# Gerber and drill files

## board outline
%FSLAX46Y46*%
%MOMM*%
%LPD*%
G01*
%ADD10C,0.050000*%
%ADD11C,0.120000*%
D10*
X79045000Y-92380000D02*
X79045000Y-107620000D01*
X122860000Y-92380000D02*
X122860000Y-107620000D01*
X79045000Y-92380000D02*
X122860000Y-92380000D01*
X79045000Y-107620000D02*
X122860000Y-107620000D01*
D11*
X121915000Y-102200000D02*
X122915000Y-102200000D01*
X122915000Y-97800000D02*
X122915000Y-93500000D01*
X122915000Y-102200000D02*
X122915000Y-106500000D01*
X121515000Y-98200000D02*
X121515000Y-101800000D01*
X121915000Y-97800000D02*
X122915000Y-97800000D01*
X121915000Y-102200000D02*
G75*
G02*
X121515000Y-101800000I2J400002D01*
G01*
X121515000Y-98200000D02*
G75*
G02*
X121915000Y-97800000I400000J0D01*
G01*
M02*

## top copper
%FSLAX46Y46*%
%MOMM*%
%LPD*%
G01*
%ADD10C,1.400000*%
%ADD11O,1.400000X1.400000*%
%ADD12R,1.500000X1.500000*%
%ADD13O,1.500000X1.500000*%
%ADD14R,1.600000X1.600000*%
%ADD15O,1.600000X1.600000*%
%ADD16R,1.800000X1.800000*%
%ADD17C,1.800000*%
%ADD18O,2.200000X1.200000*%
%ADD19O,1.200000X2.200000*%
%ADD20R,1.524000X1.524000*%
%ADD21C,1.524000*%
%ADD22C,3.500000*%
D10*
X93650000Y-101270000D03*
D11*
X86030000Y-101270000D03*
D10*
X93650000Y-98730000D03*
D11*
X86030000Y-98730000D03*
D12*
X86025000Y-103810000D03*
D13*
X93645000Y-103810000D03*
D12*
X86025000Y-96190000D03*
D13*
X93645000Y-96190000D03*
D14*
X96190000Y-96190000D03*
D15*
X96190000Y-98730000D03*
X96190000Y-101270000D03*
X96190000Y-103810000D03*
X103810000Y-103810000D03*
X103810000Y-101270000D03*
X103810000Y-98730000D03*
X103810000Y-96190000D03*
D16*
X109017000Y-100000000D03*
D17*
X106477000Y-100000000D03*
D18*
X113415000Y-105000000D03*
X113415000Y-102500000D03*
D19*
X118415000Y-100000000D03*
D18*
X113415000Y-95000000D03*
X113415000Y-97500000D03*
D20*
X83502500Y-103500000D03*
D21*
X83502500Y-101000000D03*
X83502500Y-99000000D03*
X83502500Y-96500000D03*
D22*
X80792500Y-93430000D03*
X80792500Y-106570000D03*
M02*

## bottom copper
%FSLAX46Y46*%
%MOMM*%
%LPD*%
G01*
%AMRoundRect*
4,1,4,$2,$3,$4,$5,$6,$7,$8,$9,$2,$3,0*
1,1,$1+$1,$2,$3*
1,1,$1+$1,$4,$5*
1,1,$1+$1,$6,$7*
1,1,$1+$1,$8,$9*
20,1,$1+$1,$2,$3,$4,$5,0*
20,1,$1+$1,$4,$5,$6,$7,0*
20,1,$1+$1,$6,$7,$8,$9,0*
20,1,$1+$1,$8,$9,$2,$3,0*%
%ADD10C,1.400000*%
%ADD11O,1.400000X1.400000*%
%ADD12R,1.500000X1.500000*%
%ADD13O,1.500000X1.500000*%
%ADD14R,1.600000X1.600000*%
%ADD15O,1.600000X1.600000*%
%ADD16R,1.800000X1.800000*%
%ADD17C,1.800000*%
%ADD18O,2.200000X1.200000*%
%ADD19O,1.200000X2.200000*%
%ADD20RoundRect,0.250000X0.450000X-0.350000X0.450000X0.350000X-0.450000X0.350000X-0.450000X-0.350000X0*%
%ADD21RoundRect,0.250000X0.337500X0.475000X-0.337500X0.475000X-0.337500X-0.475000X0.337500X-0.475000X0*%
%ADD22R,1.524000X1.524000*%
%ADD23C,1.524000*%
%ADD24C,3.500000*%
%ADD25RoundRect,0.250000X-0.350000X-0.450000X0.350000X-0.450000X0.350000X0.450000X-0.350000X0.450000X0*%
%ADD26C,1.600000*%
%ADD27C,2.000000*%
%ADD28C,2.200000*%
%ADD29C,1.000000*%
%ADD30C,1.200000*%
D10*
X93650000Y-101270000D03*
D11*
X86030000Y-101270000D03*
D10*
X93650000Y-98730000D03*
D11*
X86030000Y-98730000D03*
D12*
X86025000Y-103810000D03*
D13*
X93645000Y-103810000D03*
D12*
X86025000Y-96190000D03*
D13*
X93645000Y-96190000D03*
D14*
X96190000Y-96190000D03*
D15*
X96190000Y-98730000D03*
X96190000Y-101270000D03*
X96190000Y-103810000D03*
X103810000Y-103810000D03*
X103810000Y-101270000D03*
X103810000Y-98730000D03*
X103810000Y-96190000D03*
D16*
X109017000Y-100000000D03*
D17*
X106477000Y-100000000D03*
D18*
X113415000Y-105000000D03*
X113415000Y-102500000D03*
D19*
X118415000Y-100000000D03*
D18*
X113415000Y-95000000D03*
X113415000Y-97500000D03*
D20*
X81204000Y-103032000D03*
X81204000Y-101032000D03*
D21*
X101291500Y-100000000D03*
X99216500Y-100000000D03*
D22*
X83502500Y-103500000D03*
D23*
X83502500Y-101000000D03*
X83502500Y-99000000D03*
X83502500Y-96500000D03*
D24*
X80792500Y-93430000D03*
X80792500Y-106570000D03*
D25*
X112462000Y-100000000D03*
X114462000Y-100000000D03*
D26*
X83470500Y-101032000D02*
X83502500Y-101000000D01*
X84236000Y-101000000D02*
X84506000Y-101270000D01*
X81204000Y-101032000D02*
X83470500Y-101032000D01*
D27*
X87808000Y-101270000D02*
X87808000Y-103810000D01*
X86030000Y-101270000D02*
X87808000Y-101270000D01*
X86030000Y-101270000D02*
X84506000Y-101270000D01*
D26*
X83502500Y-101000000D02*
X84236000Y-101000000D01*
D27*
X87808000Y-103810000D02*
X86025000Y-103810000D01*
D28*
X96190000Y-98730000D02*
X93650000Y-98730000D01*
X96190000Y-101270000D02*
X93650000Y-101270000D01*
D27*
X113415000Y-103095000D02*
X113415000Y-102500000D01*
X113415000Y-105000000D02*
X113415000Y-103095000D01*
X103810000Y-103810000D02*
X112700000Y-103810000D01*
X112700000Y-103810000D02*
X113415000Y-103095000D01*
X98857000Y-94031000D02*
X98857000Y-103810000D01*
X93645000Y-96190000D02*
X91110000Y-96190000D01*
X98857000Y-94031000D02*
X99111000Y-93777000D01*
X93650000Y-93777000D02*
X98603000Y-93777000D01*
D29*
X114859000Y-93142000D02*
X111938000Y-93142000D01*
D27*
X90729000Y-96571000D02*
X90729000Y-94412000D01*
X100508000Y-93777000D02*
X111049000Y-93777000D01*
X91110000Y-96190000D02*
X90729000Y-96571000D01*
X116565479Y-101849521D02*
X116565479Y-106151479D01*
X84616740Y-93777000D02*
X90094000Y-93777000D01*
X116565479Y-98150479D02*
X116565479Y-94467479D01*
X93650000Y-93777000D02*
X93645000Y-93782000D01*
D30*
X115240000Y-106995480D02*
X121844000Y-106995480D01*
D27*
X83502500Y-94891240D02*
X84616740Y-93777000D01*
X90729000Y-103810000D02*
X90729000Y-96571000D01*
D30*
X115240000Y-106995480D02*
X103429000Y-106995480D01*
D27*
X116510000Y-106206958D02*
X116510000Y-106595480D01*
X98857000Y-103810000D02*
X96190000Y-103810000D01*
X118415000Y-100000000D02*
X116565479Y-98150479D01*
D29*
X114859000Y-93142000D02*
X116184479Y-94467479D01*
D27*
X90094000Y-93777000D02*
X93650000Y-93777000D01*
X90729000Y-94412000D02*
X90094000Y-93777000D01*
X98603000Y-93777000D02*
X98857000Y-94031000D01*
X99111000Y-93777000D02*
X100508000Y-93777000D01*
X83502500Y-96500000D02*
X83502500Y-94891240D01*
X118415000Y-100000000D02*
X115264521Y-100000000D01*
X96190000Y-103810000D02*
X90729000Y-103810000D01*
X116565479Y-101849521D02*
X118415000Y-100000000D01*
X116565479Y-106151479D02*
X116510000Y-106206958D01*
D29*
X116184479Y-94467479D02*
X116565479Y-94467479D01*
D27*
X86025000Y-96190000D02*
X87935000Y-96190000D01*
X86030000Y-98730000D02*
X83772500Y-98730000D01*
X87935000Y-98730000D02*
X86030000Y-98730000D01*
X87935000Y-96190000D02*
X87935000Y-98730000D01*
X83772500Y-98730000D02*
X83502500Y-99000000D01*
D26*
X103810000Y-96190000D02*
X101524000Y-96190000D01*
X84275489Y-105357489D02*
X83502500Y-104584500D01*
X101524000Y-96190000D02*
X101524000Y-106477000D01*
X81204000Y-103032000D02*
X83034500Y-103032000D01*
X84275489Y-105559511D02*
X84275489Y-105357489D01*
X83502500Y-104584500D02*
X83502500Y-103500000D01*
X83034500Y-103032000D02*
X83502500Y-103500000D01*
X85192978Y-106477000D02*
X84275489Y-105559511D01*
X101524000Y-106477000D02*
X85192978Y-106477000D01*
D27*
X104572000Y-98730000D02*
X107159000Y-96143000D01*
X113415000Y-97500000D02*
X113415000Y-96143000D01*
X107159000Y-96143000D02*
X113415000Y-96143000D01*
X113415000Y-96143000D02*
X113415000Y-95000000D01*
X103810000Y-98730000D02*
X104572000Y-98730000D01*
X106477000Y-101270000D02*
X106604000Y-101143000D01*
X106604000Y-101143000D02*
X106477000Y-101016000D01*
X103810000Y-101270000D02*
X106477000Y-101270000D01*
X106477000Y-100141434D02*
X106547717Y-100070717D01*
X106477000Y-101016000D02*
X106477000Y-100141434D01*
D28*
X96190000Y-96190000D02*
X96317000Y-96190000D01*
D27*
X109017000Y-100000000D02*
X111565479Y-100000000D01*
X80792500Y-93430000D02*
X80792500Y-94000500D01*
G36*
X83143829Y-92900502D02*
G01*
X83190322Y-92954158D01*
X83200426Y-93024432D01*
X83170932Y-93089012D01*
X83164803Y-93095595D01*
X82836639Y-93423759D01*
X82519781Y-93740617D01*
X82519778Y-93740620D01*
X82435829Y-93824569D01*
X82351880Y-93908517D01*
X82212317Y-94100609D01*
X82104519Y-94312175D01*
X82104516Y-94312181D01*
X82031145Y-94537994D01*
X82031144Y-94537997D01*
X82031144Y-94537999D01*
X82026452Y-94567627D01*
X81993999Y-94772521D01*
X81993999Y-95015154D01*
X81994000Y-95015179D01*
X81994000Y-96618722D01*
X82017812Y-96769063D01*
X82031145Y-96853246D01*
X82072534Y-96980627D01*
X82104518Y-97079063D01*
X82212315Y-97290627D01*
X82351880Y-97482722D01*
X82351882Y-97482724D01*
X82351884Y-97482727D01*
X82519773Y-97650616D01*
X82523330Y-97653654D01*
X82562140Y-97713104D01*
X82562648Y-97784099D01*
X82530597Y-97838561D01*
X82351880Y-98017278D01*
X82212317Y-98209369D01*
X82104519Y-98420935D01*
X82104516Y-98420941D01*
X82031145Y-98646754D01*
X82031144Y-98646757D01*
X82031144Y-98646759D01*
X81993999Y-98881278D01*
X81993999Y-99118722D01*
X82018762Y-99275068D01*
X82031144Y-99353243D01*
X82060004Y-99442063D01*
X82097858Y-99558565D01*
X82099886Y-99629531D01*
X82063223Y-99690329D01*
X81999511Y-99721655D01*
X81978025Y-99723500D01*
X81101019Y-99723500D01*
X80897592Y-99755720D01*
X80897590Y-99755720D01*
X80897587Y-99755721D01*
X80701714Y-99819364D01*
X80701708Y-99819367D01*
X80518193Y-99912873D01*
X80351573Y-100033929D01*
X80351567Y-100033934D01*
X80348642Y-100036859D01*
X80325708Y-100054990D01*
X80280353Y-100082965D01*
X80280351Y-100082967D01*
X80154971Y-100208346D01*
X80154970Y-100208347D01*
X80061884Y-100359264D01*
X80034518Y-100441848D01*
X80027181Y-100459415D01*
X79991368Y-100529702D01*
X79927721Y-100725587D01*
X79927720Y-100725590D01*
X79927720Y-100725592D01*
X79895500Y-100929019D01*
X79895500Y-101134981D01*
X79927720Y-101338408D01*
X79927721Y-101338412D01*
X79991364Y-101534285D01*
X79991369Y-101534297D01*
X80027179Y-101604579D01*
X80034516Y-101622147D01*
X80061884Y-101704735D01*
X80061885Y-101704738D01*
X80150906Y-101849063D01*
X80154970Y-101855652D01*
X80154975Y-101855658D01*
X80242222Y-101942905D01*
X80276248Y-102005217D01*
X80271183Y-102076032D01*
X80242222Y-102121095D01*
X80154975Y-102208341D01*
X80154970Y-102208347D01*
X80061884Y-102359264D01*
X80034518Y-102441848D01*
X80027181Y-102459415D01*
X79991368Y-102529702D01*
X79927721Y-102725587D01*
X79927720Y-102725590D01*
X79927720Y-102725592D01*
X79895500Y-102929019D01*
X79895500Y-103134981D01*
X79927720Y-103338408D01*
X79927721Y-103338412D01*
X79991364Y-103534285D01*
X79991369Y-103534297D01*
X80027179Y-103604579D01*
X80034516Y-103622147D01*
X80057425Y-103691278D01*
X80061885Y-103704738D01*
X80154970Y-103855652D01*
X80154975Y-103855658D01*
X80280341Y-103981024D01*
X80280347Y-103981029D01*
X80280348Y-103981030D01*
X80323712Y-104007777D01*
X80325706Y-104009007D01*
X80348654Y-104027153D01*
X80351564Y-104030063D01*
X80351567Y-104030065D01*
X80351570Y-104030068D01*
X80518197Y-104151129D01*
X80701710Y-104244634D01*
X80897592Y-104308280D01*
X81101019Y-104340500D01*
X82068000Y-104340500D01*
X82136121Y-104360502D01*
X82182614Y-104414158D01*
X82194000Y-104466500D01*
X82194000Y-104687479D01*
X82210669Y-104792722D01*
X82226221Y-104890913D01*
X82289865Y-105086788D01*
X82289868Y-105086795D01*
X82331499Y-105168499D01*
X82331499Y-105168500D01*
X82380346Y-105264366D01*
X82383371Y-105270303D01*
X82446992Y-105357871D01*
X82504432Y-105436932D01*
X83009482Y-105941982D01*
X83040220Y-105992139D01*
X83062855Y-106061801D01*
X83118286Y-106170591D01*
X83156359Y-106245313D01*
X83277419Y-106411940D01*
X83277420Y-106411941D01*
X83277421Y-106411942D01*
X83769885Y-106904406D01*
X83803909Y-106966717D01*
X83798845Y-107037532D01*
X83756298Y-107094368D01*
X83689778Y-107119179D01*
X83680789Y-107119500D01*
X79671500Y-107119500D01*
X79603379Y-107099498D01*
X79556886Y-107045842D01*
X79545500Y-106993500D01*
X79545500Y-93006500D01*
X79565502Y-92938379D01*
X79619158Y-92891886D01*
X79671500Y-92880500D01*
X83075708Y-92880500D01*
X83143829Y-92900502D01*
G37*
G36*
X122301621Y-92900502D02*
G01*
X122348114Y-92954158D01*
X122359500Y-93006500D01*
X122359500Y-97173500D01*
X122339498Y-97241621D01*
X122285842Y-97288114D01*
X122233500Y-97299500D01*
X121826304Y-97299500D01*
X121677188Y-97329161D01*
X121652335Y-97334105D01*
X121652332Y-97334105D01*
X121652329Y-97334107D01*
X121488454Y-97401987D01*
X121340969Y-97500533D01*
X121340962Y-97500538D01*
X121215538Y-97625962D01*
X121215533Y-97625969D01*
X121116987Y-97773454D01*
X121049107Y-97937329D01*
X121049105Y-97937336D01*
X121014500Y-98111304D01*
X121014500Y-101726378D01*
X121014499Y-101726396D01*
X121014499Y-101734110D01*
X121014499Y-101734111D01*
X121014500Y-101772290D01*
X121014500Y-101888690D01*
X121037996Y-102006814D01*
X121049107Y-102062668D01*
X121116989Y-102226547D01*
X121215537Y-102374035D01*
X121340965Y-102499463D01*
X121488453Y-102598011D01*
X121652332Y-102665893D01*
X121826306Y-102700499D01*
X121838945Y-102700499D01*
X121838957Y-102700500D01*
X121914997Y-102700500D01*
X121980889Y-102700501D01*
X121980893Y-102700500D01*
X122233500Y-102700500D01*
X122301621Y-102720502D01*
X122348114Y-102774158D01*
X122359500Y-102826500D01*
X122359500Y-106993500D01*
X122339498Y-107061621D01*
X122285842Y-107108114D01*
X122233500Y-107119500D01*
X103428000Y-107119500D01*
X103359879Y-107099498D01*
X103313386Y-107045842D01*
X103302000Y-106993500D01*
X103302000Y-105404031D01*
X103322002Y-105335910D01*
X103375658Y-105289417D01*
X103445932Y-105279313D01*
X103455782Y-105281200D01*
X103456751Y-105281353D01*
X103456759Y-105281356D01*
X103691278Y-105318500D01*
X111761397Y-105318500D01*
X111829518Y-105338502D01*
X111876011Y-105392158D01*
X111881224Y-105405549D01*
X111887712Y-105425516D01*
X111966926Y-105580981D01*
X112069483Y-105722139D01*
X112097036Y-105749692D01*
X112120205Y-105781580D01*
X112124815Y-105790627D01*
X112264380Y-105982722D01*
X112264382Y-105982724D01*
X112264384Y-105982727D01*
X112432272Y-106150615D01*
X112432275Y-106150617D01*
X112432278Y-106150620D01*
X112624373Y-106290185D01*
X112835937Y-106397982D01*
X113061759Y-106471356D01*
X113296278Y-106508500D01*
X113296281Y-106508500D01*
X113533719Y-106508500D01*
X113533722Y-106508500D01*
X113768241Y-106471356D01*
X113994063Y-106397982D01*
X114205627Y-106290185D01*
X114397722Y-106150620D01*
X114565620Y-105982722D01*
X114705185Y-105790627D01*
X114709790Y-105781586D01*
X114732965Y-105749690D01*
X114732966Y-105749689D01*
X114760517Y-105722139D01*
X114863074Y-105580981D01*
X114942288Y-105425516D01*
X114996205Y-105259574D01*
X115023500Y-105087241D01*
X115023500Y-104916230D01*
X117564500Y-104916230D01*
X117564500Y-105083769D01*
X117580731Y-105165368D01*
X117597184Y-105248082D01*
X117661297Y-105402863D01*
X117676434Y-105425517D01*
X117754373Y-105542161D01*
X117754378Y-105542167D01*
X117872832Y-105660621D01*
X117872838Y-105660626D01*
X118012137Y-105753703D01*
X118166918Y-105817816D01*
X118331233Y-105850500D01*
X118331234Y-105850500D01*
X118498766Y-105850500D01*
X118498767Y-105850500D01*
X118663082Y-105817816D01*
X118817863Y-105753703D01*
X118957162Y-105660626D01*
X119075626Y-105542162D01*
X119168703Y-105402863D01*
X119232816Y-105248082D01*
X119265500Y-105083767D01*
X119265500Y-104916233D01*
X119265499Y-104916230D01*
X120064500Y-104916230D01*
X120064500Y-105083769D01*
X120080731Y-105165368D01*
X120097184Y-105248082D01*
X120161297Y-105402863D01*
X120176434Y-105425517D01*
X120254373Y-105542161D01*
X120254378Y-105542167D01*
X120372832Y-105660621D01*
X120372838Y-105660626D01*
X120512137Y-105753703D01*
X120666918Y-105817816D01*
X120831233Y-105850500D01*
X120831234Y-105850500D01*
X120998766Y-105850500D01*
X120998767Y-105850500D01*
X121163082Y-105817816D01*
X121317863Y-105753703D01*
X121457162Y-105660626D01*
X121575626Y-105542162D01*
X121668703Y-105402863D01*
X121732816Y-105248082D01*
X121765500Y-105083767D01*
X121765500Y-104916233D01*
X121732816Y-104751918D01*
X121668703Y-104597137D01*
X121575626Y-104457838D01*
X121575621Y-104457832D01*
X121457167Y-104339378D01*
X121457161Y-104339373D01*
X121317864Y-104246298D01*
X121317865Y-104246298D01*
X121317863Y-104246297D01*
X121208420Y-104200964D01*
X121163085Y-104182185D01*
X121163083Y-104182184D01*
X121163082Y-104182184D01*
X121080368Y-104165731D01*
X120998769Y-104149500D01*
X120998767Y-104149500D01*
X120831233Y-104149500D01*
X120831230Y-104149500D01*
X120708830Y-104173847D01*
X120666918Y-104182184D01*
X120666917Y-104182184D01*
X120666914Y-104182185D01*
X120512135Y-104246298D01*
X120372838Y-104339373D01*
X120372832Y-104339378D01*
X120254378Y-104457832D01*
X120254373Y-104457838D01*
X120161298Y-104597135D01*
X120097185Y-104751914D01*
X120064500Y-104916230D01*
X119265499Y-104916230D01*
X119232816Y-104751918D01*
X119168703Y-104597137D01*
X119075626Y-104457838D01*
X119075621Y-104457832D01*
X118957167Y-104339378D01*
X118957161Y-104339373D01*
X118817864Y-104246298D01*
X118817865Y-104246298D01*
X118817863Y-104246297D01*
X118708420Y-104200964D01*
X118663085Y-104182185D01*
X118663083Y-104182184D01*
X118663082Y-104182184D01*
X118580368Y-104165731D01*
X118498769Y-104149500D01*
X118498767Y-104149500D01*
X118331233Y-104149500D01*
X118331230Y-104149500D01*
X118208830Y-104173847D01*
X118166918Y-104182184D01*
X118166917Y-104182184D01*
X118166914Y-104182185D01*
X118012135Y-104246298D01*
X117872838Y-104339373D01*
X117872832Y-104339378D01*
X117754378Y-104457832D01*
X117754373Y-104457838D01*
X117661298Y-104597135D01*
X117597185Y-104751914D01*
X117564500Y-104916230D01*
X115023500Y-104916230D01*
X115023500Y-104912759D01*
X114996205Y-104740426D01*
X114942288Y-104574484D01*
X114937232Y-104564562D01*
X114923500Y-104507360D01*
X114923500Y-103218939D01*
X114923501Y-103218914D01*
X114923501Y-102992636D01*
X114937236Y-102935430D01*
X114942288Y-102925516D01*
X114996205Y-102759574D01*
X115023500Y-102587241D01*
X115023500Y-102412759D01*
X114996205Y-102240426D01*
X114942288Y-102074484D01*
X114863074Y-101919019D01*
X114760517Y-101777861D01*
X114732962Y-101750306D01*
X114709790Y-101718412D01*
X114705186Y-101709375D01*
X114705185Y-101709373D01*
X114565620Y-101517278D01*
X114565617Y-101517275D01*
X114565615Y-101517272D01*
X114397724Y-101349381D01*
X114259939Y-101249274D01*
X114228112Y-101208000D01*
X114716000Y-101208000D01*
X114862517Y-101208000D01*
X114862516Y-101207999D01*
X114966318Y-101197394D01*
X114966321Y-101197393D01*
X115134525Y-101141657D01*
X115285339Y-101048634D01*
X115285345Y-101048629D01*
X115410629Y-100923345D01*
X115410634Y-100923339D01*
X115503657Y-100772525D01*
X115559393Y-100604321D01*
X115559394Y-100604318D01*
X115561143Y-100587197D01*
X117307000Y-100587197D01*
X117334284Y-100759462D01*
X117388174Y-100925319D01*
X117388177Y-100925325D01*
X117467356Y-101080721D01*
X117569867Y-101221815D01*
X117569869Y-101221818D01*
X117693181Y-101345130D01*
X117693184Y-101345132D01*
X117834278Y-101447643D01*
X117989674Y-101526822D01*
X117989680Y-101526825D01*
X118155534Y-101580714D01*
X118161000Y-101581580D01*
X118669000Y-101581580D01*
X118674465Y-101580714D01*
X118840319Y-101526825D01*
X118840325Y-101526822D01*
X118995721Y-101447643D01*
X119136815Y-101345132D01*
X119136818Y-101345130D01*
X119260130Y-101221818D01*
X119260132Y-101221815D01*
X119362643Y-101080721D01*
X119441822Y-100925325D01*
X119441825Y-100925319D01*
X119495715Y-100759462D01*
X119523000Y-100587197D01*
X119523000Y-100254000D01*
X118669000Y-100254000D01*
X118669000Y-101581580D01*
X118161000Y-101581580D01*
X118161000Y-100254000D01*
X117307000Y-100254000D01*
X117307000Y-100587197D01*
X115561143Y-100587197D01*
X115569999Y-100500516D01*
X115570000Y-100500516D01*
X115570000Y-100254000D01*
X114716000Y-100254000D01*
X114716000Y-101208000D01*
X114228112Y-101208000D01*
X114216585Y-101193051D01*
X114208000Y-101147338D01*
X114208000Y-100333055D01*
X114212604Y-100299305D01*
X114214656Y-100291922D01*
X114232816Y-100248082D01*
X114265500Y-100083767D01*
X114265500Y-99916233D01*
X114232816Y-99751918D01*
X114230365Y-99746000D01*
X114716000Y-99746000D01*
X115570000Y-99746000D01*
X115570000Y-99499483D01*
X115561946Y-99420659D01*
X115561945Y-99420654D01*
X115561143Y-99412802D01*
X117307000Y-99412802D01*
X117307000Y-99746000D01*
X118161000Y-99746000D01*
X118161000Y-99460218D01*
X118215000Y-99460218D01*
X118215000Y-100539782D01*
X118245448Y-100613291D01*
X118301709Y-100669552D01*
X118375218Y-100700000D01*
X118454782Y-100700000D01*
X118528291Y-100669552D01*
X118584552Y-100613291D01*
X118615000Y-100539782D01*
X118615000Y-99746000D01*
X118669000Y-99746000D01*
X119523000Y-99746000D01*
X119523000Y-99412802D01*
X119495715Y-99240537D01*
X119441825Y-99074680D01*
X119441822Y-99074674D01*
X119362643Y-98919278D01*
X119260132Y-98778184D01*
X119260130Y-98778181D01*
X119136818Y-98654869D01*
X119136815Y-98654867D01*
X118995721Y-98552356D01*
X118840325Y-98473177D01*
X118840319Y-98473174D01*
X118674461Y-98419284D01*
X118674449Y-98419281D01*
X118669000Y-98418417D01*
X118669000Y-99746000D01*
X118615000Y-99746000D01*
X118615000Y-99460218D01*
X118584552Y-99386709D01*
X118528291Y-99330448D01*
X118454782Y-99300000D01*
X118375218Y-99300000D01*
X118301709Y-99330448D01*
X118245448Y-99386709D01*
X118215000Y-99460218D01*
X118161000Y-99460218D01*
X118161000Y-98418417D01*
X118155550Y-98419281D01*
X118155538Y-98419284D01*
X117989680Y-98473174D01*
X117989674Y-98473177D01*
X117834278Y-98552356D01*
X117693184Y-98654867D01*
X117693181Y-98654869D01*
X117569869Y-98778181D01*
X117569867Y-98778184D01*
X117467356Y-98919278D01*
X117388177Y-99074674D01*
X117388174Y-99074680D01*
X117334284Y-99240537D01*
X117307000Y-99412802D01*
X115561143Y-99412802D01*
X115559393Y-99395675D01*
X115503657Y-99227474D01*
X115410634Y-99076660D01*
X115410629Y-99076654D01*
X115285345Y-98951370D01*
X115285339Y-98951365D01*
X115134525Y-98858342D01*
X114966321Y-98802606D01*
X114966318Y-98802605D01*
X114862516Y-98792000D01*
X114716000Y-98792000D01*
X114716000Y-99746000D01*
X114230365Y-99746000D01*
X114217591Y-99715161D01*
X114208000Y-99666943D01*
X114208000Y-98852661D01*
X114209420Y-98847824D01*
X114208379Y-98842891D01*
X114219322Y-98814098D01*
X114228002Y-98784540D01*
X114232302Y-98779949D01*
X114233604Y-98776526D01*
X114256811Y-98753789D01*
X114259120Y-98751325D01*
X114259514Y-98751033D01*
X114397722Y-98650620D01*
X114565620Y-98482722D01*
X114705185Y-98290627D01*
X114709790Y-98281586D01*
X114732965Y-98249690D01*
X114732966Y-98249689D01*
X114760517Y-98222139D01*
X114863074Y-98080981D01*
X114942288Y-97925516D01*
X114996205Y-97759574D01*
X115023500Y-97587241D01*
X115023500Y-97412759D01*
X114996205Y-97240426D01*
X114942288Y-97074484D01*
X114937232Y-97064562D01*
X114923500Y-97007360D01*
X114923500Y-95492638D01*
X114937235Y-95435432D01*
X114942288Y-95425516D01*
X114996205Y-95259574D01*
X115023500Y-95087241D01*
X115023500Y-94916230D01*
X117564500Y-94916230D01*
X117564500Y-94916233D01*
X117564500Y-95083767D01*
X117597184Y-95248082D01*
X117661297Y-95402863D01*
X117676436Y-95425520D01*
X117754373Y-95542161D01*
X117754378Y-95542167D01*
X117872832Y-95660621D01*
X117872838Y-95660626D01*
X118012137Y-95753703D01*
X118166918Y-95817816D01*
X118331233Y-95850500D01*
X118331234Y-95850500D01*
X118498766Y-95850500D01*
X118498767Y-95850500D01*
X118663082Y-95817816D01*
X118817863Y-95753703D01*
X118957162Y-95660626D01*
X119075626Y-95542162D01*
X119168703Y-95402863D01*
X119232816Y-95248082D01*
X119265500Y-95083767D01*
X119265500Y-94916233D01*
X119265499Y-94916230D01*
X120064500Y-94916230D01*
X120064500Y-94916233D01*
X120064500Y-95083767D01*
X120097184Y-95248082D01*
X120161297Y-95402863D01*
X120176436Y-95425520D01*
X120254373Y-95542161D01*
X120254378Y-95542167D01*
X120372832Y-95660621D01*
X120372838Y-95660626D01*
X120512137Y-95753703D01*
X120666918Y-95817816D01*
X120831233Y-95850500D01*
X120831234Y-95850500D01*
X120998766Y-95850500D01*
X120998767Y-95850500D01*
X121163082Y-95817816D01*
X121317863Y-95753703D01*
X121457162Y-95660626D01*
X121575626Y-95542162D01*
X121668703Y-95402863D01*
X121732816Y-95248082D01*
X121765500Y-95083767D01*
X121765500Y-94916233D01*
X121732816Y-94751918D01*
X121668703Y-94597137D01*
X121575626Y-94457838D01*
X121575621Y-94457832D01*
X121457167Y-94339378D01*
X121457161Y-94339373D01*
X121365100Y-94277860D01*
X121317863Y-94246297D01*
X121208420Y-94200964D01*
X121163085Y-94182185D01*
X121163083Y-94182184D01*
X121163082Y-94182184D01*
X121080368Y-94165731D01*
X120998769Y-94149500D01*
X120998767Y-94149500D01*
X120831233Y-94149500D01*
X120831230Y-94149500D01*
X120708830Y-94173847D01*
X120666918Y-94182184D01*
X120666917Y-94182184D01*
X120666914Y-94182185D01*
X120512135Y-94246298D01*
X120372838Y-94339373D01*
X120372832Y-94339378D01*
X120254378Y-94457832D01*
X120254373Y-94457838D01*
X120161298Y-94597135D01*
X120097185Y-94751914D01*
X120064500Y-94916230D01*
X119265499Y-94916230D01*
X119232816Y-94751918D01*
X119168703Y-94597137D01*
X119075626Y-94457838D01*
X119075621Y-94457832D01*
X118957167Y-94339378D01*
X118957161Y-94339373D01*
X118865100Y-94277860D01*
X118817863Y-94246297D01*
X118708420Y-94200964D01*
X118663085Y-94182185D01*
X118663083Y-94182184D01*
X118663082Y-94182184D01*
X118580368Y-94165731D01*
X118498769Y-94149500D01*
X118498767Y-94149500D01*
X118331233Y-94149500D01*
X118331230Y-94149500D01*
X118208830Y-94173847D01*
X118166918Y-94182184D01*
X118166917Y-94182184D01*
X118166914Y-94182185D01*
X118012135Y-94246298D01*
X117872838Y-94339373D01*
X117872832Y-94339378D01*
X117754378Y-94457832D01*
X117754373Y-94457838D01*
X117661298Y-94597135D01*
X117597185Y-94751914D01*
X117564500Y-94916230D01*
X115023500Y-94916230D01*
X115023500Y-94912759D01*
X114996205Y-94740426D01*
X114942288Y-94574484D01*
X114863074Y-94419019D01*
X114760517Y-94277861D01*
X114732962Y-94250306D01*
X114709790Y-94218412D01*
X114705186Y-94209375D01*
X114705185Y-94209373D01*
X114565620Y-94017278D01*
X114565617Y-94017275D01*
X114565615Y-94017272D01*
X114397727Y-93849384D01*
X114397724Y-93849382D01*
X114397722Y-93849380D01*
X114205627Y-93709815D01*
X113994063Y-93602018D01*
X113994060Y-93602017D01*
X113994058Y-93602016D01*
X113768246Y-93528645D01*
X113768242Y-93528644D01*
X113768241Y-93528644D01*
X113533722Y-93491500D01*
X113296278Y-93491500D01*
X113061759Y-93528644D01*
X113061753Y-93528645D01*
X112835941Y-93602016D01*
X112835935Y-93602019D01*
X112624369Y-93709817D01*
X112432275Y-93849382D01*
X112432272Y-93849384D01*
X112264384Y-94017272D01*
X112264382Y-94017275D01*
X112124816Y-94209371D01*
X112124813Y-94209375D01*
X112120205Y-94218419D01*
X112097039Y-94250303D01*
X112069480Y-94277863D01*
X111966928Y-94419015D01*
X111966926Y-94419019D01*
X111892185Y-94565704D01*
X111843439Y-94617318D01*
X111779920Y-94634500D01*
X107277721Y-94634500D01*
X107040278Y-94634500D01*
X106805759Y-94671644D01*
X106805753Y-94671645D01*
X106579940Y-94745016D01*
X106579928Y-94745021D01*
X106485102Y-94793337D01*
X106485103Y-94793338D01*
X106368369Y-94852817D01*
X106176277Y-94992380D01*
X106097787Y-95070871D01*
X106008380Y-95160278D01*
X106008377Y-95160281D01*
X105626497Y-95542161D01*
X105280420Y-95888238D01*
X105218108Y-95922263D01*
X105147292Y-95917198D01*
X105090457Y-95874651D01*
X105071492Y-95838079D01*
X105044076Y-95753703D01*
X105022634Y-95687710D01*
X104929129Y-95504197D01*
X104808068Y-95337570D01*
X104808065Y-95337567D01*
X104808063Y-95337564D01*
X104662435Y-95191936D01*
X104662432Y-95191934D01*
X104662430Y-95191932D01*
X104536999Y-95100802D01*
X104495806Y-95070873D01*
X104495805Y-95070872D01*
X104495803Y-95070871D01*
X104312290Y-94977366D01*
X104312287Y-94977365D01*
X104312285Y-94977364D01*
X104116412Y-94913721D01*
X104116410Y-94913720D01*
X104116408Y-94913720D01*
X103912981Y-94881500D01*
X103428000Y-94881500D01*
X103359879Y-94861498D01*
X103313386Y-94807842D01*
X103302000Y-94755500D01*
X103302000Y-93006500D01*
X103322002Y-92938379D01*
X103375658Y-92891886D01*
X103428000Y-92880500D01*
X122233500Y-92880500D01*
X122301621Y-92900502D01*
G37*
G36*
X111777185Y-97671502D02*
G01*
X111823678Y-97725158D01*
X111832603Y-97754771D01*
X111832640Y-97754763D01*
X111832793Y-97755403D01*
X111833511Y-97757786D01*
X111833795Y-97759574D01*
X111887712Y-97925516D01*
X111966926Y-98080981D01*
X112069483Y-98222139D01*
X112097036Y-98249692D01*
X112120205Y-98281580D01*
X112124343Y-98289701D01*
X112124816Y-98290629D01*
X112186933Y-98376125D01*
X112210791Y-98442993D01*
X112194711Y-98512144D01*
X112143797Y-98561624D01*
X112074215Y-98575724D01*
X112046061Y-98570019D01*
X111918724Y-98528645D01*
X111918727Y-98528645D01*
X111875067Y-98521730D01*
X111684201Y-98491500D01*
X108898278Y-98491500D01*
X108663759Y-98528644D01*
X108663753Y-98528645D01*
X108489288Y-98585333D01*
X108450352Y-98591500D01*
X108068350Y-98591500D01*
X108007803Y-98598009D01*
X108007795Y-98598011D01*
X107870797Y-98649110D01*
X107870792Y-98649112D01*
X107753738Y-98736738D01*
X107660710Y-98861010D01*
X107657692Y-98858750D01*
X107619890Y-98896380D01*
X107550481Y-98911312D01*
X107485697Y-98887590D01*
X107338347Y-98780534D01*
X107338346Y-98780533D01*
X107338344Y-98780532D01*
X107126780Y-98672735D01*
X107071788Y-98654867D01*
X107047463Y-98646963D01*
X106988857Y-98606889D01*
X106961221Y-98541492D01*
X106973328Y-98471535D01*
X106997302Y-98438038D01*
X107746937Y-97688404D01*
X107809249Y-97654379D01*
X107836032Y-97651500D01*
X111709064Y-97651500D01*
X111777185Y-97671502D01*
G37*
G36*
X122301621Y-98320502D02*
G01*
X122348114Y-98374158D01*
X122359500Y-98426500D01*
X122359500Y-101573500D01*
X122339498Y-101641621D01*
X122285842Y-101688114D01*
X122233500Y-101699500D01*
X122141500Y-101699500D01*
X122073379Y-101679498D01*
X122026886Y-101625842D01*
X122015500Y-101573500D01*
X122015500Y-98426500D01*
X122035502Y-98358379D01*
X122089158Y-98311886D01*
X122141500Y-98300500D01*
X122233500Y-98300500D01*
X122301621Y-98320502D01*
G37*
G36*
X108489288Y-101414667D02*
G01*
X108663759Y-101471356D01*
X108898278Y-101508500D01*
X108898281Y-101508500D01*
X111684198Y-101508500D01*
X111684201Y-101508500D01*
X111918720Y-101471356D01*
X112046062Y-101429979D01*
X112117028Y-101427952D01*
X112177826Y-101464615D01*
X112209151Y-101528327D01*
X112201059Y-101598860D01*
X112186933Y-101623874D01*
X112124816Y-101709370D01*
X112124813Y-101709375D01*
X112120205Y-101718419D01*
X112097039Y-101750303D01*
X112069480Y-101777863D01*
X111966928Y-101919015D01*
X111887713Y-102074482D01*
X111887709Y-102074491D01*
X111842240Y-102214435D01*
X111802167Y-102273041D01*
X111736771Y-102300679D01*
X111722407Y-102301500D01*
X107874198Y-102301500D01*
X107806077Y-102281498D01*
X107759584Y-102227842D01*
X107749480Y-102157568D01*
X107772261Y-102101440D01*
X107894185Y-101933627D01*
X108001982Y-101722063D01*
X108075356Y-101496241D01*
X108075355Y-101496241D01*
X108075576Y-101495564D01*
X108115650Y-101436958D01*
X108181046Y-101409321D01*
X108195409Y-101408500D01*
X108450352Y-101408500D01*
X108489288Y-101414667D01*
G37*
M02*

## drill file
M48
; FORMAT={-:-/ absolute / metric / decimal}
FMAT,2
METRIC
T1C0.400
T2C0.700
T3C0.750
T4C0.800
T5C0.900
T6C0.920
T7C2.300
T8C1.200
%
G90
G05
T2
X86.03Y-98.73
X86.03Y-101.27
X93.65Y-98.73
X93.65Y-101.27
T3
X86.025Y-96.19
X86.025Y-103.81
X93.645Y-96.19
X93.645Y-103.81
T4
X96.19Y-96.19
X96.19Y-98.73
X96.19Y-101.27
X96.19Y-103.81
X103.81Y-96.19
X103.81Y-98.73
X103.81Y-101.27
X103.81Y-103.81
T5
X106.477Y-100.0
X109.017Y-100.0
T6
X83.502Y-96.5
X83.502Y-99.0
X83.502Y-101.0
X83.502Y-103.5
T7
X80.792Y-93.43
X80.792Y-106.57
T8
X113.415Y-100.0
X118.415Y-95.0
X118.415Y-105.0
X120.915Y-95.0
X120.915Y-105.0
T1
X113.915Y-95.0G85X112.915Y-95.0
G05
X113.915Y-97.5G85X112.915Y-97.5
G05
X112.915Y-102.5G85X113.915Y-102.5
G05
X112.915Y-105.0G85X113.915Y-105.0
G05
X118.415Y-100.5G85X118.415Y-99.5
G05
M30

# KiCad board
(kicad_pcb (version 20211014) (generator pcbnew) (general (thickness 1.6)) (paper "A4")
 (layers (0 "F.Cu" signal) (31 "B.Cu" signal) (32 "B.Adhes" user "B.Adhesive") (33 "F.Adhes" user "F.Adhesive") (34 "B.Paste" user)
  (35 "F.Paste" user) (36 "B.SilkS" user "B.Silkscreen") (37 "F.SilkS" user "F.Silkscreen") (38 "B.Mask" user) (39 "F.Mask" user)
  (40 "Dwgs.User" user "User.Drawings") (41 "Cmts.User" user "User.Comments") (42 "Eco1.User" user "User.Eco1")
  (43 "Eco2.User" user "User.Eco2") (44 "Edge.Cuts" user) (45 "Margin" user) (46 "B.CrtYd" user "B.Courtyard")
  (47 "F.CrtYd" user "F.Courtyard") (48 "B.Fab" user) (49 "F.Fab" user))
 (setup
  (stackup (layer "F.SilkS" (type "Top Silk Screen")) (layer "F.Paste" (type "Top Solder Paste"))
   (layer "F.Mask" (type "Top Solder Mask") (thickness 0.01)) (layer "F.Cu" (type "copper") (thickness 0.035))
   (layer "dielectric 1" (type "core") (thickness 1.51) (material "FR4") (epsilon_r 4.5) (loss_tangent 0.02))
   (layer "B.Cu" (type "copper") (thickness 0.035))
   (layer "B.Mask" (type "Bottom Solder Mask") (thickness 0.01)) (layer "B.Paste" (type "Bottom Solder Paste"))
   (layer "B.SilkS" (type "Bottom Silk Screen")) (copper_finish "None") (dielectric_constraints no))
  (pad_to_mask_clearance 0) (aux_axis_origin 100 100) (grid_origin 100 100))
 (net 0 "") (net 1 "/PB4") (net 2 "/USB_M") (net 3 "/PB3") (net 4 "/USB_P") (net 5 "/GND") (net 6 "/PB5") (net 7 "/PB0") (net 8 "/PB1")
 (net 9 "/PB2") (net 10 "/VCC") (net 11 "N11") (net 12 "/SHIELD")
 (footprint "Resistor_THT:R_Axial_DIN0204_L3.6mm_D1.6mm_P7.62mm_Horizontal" (layer "F.Cu") (at 93.65 101.27 180)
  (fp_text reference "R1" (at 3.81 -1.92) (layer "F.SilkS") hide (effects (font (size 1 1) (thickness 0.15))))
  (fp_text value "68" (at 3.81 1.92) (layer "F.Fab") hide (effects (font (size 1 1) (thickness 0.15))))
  (pad "1" thru_hole circle locked (at 0 0 180) (size 1.4 1.4) (drill 0.7) (layers *.Cu *.Mask) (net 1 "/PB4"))
  (pad "2" thru_hole oval locked (at 7.62 0 180) (size 1.4 1.4) (drill 0.7) (layers *.Cu *.Mask) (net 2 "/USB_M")))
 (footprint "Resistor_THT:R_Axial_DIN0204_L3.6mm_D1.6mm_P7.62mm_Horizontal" (layer "F.Cu") (at 93.65 98.73 180)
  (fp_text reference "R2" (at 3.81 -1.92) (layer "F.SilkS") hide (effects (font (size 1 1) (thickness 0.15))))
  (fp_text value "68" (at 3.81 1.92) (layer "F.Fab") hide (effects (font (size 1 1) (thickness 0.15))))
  (pad "1" thru_hole circle locked (at 0 0 180) (size 1.4 1.4) (drill 0.7) (layers *.Cu *.Mask) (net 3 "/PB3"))
  (pad "2" thru_hole oval locked (at 7.62 0 180) (size 1.4 1.4) (drill 0.7) (layers *.Cu *.Mask) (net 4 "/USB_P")))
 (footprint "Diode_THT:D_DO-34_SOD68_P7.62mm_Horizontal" (layer "F.Cu") (at 86.025 103.81)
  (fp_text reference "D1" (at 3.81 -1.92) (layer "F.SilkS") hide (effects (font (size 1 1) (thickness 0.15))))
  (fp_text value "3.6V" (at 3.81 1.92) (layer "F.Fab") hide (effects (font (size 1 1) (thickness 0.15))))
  (pad "1" thru_hole rect locked (at 0 0) (size 1.5 1.5) (drill 0.75) (layers *.Cu *.Mask) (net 2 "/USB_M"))
  (pad "2" thru_hole oval locked (at 7.62 0) (size 1.5 1.5) (drill 0.75) (layers *.Cu *.Mask) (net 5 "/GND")))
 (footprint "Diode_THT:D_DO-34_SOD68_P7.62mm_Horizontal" (layer "F.Cu") (at 86.025 96.19)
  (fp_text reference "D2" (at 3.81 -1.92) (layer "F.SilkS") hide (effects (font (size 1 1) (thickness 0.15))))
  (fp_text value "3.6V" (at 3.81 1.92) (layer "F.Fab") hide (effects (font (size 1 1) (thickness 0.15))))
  (pad "1" thru_hole rect locked (at 0 0) (size 1.5 1.5) (drill 0.75) (layers *.Cu *.Mask) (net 4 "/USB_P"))
  (pad "2" thru_hole oval locked (at 7.62 0) (size 1.5 1.5) (drill 0.75) (layers *.Cu *.Mask) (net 5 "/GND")))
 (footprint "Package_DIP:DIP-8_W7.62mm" (layer "F.Cu") (at 96.19 96.19)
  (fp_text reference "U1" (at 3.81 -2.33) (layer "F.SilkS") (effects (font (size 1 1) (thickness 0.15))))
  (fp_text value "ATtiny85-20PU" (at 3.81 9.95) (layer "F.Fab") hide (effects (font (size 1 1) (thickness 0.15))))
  (pad "1" thru_hole rect locked (at 0 0) (size 1.6 1.6) (drill 0.8) (layers *.Cu *.Mask) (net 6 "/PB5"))
  (pad "2" thru_hole oval locked (at 0 2.54) (size 1.6 1.6) (drill 0.8) (layers *.Cu *.Mask) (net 3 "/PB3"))
  (pad "3" thru_hole oval locked (at 0 5.08) (size 1.6 1.6) (drill 0.8) (layers *.Cu *.Mask) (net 1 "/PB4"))
  (pad "4" thru_hole oval locked (at 0 7.62) (size 1.6 1.6) (drill 0.8) (layers *.Cu *.Mask) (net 5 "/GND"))
  (pad "5" thru_hole oval locked (at 7.62 7.62) (size 1.6 1.6) (drill 0.8) (layers *.Cu *.Mask) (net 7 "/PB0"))
  (pad "6" thru_hole oval locked (at 7.62 5.08) (size 1.6 1.6) (drill 0.8) (layers *.Cu *.Mask) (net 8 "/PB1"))
  (pad "7" thru_hole oval locked (at 7.62 2.54) (size 1.6 1.6) (drill 0.8) (layers *.Cu *.Mask) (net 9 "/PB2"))
  (pad "8" thru_hole oval locked (at 7.62 0) (size 1.6 1.6) (drill 0.8) (layers *.Cu *.Mask) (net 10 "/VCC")))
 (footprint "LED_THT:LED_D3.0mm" (layer "F.Cu") (at 109.017 100 180)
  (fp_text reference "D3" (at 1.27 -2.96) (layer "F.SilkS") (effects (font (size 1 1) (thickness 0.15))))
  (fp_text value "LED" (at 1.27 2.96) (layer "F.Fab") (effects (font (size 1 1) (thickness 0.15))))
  (pad "1" thru_hole rect (at 0 0 180) (size 1.8 1.8) (drill 0.9) (layers *.Cu *.Mask) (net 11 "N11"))
  (pad "2" thru_hole circle (at 2.54 0 180) (size 1.8 1.8) (drill 0.9) (layers *.Cu *.Mask) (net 8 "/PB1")))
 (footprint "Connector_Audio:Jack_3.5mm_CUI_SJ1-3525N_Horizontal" (layer "F.Cu") (at 118.415 100 90)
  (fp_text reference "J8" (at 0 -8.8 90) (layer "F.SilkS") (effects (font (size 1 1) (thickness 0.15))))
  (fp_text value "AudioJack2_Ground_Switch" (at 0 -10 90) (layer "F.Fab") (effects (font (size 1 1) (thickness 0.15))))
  (fp_line (start -2.2 3.5) (end -2.2 4.5) (layer "Edge.Cuts") (width 0.12))
  (fp_line (start 2.2 4.5) (end 6.5 4.5) (layer "Edge.Cuts") (width 0.12))
  (fp_line (start -2.2 4.5) (end -6.5 4.5) (layer "Edge.Cuts") (width 0.12))
  (fp_line (start 1.8 3.1) (end -1.8 3.1) (layer "Edge.Cuts") (width 0.12))
  (fp_line (start 2.2 3.5) (end 2.2 4.5) (layer "Edge.Cuts") (width 0.12))
  (fp_arc (start -2.2 3.5) (mid -2.082842 3.217158) (end -1.8 3.1) (layer "Edge.Cuts") (width 0.12))
  (fp_arc (start 1.8 3.1) (mid 2.082843 3.217157) (end 2.2 3.5) (layer "Edge.Cuts") (width 0.12))
  (pad "" np_thru_hole circle (at 5 2.5 90) (size 1.2 1.2) (drill 1.2) (layers *.Cu))
  (pad "" np_thru_hole circle (at 5 0 90) (size 1.2 1.2) (drill 1.2) (layers *.Cu))
  (pad "" np_thru_hole circle (at -5 2.5 90) (size 1.2 1.2) (drill 1.2) (layers *.Cu))
  (pad "" np_thru_hole circle (at -5 0 90) (size 1.2 1.2) (drill 1.2) (layers *.Cu))
  (pad "" np_thru_hole circle (at 0 -5 90) (size 1.2 1.2) (drill 1.2) (layers *.Cu))
  (pad "R" thru_hole oval (at -5 -5 90) (size 1.2 2.2) (drill oval 0.4 1.4) (layers *.Cu *.Mask) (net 7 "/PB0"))
  (pad "RN" thru_hole oval (at -2.5 -5 90) (size 1.2 2.2) (drill oval 0.4 1.4) (layers *.Cu *.Mask) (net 7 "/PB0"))
  (pad "S" thru_hole oval (at 0 0 90) (size 2.2 1.2) (drill oval 1.4 0.4) (layers *.Cu *.Mask) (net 5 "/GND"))
  (pad "T" thru_hole oval (at 5 -5 270) (size 1.2 2.2) (drill oval 0.4 1.4) (layers *.Cu *.Mask) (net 9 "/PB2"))
  (pad "TN" thru_hole oval (at 2.5 -5 270) (size 1.2 2.2) (drill oval 0.4 1.4) (layers *.Cu *.Mask) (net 9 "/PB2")))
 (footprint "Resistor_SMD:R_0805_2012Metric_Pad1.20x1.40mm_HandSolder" (layer "B.Cu") (at 81.204 102.032 90)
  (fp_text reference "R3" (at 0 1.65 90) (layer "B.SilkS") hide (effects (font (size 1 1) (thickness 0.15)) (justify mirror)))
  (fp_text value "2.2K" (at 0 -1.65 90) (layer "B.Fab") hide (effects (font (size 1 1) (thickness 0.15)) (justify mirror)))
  (pad "1" smd roundrect locked (at -1 0 90) (size 1.2 1.4) (layers "B.Cu" "B.Paste" "B.Mask") (roundrect_rratio 0.2083333333)
   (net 10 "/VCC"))
  (pad "2" smd roundrect locked (at 1 0 90) (size 1.2 1.4) (layers "B.Cu" "B.Paste" "B.Mask") (roundrect_rratio 0.2083333333)
   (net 2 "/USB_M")))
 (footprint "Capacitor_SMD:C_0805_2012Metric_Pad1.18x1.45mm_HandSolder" (layer "B.Cu") (at 100.254 100 180)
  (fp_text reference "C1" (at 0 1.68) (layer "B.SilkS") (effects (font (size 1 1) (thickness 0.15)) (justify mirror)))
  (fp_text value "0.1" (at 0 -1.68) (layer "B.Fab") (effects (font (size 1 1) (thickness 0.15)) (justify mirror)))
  (pad "1" smd roundrect locked (at -1.0375 0 180) (size 1.175 1.45) (layers "B.Cu" "B.Paste" "B.Mask") (roundrect_rratio 0.2127659574)
   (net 10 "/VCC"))
  (pad "2" smd roundrect locked (at 1.0375 0 180) (size 1.175 1.45) (layers "B.Cu" "B.Paste" "B.Mask") (roundrect_rratio 0.2127659574)
   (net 5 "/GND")))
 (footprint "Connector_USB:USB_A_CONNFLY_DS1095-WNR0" (layer "B.Cu") (at 83.5025 103.5 90)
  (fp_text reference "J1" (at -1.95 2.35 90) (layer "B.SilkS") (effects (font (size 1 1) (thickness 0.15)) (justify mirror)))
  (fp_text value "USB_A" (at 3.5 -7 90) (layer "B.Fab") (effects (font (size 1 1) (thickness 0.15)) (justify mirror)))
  (pad "1" thru_hole rect (at 0 0 90) (size 1.524 1.524) (drill 0.92) (layers *.Cu *.Mask) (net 10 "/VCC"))
  (pad "2" thru_hole circle (at 2.5 0 90) (size 1.524 1.524) (drill 0.92) (layers *.Cu *.Mask) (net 2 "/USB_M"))
  (pad "3" thru_hole circle (at 4.5 0 90) (size 1.524 1.524) (drill 0.92) (layers *.Cu *.Mask) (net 4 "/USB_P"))
  (pad "4" thru_hole circle (at 7 0 90) (size 1.524 1.524) (drill 0.92) (layers *.Cu *.Mask) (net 5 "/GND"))
  (pad "5" thru_hole circle (at 10.07 -2.71 90) (size 3.5 3.5) (drill 2.3) (layers *.Cu *.Mask) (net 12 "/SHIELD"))
  (pad "5" thru_hole circle (at -3.07 -2.71 90) (size 3.5 3.5) (drill 2.3) (layers *.Cu *.Mask) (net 12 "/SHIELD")))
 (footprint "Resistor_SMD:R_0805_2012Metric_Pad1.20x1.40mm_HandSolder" (layer "B.Cu") (at 113.462 100)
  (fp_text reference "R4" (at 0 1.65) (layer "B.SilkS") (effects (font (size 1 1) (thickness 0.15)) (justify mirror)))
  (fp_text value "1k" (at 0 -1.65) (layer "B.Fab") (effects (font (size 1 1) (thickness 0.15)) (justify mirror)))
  (pad "1" smd roundrect (at -1 0) (size 1.2 1.4) (layers "B.Cu" "B.Paste" "B.Mask") (roundrect_rratio 0.208333) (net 11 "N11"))
  (pad "2" smd roundrect (at 1 0) (size 1.2 1.4) (layers "B.Cu" "B.Paste" "B.Mask") (roundrect_rratio 0.208333) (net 5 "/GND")))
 (gr_line (start 79.045 92.38) (end 79.045 107.62) (layer "Edge.Cuts") (width 0.05))
 (gr_line (start 122.86 92.38) (end 122.86 107.62) (layer "Edge.Cuts") (width 0.05))
 (gr_line (start 79.045 92.38) (end 122.86 92.38) (layer "Edge.Cuts") (width 0.05))
 (gr_line (start 79.045 107.62) (end 122.86 107.62) (layer "Edge.Cuts") (width 0.05))
 (segment (start 83.4705 101.032) (end 83.5025 101) (width 1.6) (layer "B.Cu") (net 2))
 (segment (start 84.236 101) (end 84.506 101.27) (width 1.6) (layer "B.Cu") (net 2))
 (segment (start 81.204 101.032) (end 83.4705 101.032) (width 1.6) (layer "B.Cu") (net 2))
 (segment (start 87.808 101.27) (end 87.808 103.81) (width 2) (layer "B.Cu") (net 2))
 (segment (start 86.03 101.27) (end 87.808 101.27) (width 2) (layer "B.Cu") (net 2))
 (segment (start 86.03 101.27) (end 84.506 101.27) (width 2) (layer "B.Cu") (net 2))
 (segment (start 83.5025 101) (end 84.236 101) (width 1.6) (layer "B.Cu") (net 2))
 (segment (start 87.808 103.81) (end 86.025 103.81) (width 2) (layer "B.Cu") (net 2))
 (segment (start 96.19 98.73) (end 93.65 98.73) (width 2.2) (layer "B.Cu") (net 3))
 (segment (start 96.19 101.27) (end 93.65 101.27) (width 2.2) (layer "B.Cu") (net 1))
 (segment (start 113.415 103.095) (end 113.415 102.5) (width 2) (layer "B.Cu") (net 7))
 (segment (start 113.415 105) (end 113.415 103.095) (width 2) (layer "B.Cu") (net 7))
 (segment (start 103.81 103.81) (end 112.7 103.81) (width 2) (layer "B.Cu") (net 7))
 (segment (start 112.7 103.81) (end 113.415 103.095) (width 2) (layer "B.Cu") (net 7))
 (segment (start 98.857 94.031) (end 98.857 103.81) (width 2) (layer "B.Cu") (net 5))
 (segment (start 93.645 96.19) (end 91.11 96.19) (width 2) (layer "B.Cu") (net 5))
 (segment (start 98.857 94.031) (end 99.111 93.777) (width 2) (layer "B.Cu") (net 5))
 (segment (start 93.65 93.777) (end 98.603 93.777) (width 2) (layer "B.Cu") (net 5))
 (segment (start 114.859 93.142) (end 111.938 93.142) (width 1) (layer "B.Cu") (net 5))
 (segment (start 90.729 96.571) (end 90.729 94.412) (width 2) (layer "B.Cu") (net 5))
 (segment (start 100.508 93.777) (end 111.049 93.777) (width 2) (layer "B.Cu") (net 5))
 (segment (start 91.11 96.19) (end 90.729 96.571) (width 2) (layer "B.Cu") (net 5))
 (segment (start 116.565479 101.849521) (end 116.565479 106.151479) (width 2) (layer "B.Cu") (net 5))
 (segment (start 84.61674 93.777) (end 90.094 93.777) (width 2) (layer "B.Cu") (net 5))
 (segment (start 116.565479 98.150479) (end 116.565479 94.467479) (width 2) (layer "B.Cu") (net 5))
 (segment (start 93.65 93.777) (end 93.645 93.782) (width 2) (layer "B.Cu") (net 5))
 (segment (start 115.24 106.99548) (end 121.844 106.99548) (width 1.2) (layer "B.Cu") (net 5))
 (segment (start 83.5025 94.89124) (end 84.61674 93.777) (width 2) (layer "B.Cu") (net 5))
 (segment (start 90.729 103.81) (end 90.729 96.571) (width 2) (layer "B.Cu") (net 5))
 (segment (start 115.24 106.99548) (end 103.429 106.99548) (width 1.2) (layer "B.Cu") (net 5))
 (segment (start 116.51 106.206958) (end 116.51 106.59548) (width 2) (layer "B.Cu") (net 5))
 (segment (start 98.857 103.81) (end 96.19 103.81) (width 2) (layer "B.Cu") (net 5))
 (segment (start 118.415 100) (end 116.565479 98.150479) (width 2) (layer "B.Cu") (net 5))
 (segment (start 114.859 93.142) (end 116.184479 94.467479) (width 1) (layer "B.Cu") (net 5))
 (segment (start 90.094 93.777) (end 93.65 93.777) (width 2) (layer "B.Cu") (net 5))
 (segment (start 90.729 94.412) (end 90.094 93.777) (width 2) (layer "B.Cu") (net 5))
 (segment (start 98.603 93.777) (end 98.857 94.031) (width 2) (layer "B.Cu") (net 5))
 (segment (start 99.111 93.777) (end 100.508 93.777) (width 2) (layer "B.Cu") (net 5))
 (segment (start 83.5025 96.5) (end 83.5025 94.89124) (width 2) (layer "B.Cu") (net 5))
 (segment (start 118.415 100) (end 115.264521 100) (width 2) (layer "B.Cu") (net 5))
 (segment (start 96.19 103.81) (end 90.729 103.81) (width 2) (layer "B.Cu") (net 5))
 (segment (start 116.565479 101.849521) (end 118.415 100) (width 2) (layer "B.Cu") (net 5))
 (segment (start 116.565479 106.151479) (end 116.51 106.206958) (width 2) (layer "B.Cu") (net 5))
 (segment (start 116.184479 94.467479) (end 116.565479 94.467479) (width 1) (layer "B.Cu") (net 5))
 (segment (start 86.025 96.19) (end 87.935 96.19) (width 2) (layer "B.Cu") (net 4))
 (segment (start 86.03 98.73) (end 83.7725 98.73) (width 2) (layer "B.Cu") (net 4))
 (segment (start 87.935 98.73) (end 86.03 98.73) (width 2) (layer "B.Cu") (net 4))
 (segment (start 87.935 96.19) (end 87.935 98.73) (width 2) (layer "B.Cu") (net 4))
 (segment (start 83.7725 98.73) (end 83.5025 99) (width 2) (layer "B.Cu") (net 4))
 (segment (start 103.81 96.19) (end 101.524 96.19) (width 1.6) (layer "B.Cu") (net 10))
 (segment (start 84.275489 105.357489) (end 83.5025 104.5845) (width 1.6) (layer "B.Cu") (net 10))
 (segment (start 101.524 96.19) (end 101.524 106.477) (width 1.6) (layer "B.Cu") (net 10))
 (segment (start 81.204 103.032) (end 83.0345 103.032) (width 1.6) (layer "B.Cu") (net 10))
 (segment (start 84.275489 105.559511) (end 84.275489 105.357489) (width 1.6) (layer "B.Cu") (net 10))
 (segment (start 83.5025 104.5845) (end 83.5025 103.5) (width 1.6) (layer "B.Cu") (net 10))
 (segment (start 83.0345 103.032) (end 83.5025 103.5) (width 1.6) (layer "B.Cu") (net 10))
 (segment (start 85.192978 106.477) (end 84.275489 105.559511) (width 1.6) (layer "B.Cu") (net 10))
 (segment (start 101.524 106.477) (end 85.192978 106.477) (width 1.6) (layer "B.Cu") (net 10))
 (segment (start 104.572 98.73) (end 107.159 96.143) (width 2) (layer "B.Cu") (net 9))
 (segment (start 113.415 97.5) (end 113.415 96.143) (width 2) (layer "B.Cu") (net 9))
 (segment (start 107.159 96.143) (end 113.415 96.143) (width 2) (layer "B.Cu") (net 9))
 (segment (start 113.415 96.143) (end 113.415 95) (width 2) (layer "B.Cu") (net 9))
 (segment (start 103.81 98.73) (end 104.572 98.73) (width 2) (layer "B.Cu") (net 9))
 (segment (start 106.477 101.27) (end 106.604 101.143) (width 2) (layer "B.Cu") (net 8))
 (segment (start 106.604 101.143) (end 106.477 101.016) (width 2) (layer "B.Cu") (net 8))
 (segment (start 103.81 101.27) (end 106.477 101.27) (width 2) (layer "B.Cu") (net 8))
 (segment (start 106.477 100.141434) (end 106.547717 100.070717) (width 2) (layer "B.Cu") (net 8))
 (segment (start 106.477 101.016) (end 106.477 100.141434) (width 2) (layer "B.Cu") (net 8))
 (segment (start 96.19 96.19) (end 96.317 96.19) (width 2.2) (layer "B.Cu") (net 6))
 (segment (start 109.017 100) (end 111.565479 100) (width 2) (layer "B.Cu") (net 11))
 (segment (start 80.7925 93.43) (end 80.7925 94.0005) (width 2) (layer "B.Cu") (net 12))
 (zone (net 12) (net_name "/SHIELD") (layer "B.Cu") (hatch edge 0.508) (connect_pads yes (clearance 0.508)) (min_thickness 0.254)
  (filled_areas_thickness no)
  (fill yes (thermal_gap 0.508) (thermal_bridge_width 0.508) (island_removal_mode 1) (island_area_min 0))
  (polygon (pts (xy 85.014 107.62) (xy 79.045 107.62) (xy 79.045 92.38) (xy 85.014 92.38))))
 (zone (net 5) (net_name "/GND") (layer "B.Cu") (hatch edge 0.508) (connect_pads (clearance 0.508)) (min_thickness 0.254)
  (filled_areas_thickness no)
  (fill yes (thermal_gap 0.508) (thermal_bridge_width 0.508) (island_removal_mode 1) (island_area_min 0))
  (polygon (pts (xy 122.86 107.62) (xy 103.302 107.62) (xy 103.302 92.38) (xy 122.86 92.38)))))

